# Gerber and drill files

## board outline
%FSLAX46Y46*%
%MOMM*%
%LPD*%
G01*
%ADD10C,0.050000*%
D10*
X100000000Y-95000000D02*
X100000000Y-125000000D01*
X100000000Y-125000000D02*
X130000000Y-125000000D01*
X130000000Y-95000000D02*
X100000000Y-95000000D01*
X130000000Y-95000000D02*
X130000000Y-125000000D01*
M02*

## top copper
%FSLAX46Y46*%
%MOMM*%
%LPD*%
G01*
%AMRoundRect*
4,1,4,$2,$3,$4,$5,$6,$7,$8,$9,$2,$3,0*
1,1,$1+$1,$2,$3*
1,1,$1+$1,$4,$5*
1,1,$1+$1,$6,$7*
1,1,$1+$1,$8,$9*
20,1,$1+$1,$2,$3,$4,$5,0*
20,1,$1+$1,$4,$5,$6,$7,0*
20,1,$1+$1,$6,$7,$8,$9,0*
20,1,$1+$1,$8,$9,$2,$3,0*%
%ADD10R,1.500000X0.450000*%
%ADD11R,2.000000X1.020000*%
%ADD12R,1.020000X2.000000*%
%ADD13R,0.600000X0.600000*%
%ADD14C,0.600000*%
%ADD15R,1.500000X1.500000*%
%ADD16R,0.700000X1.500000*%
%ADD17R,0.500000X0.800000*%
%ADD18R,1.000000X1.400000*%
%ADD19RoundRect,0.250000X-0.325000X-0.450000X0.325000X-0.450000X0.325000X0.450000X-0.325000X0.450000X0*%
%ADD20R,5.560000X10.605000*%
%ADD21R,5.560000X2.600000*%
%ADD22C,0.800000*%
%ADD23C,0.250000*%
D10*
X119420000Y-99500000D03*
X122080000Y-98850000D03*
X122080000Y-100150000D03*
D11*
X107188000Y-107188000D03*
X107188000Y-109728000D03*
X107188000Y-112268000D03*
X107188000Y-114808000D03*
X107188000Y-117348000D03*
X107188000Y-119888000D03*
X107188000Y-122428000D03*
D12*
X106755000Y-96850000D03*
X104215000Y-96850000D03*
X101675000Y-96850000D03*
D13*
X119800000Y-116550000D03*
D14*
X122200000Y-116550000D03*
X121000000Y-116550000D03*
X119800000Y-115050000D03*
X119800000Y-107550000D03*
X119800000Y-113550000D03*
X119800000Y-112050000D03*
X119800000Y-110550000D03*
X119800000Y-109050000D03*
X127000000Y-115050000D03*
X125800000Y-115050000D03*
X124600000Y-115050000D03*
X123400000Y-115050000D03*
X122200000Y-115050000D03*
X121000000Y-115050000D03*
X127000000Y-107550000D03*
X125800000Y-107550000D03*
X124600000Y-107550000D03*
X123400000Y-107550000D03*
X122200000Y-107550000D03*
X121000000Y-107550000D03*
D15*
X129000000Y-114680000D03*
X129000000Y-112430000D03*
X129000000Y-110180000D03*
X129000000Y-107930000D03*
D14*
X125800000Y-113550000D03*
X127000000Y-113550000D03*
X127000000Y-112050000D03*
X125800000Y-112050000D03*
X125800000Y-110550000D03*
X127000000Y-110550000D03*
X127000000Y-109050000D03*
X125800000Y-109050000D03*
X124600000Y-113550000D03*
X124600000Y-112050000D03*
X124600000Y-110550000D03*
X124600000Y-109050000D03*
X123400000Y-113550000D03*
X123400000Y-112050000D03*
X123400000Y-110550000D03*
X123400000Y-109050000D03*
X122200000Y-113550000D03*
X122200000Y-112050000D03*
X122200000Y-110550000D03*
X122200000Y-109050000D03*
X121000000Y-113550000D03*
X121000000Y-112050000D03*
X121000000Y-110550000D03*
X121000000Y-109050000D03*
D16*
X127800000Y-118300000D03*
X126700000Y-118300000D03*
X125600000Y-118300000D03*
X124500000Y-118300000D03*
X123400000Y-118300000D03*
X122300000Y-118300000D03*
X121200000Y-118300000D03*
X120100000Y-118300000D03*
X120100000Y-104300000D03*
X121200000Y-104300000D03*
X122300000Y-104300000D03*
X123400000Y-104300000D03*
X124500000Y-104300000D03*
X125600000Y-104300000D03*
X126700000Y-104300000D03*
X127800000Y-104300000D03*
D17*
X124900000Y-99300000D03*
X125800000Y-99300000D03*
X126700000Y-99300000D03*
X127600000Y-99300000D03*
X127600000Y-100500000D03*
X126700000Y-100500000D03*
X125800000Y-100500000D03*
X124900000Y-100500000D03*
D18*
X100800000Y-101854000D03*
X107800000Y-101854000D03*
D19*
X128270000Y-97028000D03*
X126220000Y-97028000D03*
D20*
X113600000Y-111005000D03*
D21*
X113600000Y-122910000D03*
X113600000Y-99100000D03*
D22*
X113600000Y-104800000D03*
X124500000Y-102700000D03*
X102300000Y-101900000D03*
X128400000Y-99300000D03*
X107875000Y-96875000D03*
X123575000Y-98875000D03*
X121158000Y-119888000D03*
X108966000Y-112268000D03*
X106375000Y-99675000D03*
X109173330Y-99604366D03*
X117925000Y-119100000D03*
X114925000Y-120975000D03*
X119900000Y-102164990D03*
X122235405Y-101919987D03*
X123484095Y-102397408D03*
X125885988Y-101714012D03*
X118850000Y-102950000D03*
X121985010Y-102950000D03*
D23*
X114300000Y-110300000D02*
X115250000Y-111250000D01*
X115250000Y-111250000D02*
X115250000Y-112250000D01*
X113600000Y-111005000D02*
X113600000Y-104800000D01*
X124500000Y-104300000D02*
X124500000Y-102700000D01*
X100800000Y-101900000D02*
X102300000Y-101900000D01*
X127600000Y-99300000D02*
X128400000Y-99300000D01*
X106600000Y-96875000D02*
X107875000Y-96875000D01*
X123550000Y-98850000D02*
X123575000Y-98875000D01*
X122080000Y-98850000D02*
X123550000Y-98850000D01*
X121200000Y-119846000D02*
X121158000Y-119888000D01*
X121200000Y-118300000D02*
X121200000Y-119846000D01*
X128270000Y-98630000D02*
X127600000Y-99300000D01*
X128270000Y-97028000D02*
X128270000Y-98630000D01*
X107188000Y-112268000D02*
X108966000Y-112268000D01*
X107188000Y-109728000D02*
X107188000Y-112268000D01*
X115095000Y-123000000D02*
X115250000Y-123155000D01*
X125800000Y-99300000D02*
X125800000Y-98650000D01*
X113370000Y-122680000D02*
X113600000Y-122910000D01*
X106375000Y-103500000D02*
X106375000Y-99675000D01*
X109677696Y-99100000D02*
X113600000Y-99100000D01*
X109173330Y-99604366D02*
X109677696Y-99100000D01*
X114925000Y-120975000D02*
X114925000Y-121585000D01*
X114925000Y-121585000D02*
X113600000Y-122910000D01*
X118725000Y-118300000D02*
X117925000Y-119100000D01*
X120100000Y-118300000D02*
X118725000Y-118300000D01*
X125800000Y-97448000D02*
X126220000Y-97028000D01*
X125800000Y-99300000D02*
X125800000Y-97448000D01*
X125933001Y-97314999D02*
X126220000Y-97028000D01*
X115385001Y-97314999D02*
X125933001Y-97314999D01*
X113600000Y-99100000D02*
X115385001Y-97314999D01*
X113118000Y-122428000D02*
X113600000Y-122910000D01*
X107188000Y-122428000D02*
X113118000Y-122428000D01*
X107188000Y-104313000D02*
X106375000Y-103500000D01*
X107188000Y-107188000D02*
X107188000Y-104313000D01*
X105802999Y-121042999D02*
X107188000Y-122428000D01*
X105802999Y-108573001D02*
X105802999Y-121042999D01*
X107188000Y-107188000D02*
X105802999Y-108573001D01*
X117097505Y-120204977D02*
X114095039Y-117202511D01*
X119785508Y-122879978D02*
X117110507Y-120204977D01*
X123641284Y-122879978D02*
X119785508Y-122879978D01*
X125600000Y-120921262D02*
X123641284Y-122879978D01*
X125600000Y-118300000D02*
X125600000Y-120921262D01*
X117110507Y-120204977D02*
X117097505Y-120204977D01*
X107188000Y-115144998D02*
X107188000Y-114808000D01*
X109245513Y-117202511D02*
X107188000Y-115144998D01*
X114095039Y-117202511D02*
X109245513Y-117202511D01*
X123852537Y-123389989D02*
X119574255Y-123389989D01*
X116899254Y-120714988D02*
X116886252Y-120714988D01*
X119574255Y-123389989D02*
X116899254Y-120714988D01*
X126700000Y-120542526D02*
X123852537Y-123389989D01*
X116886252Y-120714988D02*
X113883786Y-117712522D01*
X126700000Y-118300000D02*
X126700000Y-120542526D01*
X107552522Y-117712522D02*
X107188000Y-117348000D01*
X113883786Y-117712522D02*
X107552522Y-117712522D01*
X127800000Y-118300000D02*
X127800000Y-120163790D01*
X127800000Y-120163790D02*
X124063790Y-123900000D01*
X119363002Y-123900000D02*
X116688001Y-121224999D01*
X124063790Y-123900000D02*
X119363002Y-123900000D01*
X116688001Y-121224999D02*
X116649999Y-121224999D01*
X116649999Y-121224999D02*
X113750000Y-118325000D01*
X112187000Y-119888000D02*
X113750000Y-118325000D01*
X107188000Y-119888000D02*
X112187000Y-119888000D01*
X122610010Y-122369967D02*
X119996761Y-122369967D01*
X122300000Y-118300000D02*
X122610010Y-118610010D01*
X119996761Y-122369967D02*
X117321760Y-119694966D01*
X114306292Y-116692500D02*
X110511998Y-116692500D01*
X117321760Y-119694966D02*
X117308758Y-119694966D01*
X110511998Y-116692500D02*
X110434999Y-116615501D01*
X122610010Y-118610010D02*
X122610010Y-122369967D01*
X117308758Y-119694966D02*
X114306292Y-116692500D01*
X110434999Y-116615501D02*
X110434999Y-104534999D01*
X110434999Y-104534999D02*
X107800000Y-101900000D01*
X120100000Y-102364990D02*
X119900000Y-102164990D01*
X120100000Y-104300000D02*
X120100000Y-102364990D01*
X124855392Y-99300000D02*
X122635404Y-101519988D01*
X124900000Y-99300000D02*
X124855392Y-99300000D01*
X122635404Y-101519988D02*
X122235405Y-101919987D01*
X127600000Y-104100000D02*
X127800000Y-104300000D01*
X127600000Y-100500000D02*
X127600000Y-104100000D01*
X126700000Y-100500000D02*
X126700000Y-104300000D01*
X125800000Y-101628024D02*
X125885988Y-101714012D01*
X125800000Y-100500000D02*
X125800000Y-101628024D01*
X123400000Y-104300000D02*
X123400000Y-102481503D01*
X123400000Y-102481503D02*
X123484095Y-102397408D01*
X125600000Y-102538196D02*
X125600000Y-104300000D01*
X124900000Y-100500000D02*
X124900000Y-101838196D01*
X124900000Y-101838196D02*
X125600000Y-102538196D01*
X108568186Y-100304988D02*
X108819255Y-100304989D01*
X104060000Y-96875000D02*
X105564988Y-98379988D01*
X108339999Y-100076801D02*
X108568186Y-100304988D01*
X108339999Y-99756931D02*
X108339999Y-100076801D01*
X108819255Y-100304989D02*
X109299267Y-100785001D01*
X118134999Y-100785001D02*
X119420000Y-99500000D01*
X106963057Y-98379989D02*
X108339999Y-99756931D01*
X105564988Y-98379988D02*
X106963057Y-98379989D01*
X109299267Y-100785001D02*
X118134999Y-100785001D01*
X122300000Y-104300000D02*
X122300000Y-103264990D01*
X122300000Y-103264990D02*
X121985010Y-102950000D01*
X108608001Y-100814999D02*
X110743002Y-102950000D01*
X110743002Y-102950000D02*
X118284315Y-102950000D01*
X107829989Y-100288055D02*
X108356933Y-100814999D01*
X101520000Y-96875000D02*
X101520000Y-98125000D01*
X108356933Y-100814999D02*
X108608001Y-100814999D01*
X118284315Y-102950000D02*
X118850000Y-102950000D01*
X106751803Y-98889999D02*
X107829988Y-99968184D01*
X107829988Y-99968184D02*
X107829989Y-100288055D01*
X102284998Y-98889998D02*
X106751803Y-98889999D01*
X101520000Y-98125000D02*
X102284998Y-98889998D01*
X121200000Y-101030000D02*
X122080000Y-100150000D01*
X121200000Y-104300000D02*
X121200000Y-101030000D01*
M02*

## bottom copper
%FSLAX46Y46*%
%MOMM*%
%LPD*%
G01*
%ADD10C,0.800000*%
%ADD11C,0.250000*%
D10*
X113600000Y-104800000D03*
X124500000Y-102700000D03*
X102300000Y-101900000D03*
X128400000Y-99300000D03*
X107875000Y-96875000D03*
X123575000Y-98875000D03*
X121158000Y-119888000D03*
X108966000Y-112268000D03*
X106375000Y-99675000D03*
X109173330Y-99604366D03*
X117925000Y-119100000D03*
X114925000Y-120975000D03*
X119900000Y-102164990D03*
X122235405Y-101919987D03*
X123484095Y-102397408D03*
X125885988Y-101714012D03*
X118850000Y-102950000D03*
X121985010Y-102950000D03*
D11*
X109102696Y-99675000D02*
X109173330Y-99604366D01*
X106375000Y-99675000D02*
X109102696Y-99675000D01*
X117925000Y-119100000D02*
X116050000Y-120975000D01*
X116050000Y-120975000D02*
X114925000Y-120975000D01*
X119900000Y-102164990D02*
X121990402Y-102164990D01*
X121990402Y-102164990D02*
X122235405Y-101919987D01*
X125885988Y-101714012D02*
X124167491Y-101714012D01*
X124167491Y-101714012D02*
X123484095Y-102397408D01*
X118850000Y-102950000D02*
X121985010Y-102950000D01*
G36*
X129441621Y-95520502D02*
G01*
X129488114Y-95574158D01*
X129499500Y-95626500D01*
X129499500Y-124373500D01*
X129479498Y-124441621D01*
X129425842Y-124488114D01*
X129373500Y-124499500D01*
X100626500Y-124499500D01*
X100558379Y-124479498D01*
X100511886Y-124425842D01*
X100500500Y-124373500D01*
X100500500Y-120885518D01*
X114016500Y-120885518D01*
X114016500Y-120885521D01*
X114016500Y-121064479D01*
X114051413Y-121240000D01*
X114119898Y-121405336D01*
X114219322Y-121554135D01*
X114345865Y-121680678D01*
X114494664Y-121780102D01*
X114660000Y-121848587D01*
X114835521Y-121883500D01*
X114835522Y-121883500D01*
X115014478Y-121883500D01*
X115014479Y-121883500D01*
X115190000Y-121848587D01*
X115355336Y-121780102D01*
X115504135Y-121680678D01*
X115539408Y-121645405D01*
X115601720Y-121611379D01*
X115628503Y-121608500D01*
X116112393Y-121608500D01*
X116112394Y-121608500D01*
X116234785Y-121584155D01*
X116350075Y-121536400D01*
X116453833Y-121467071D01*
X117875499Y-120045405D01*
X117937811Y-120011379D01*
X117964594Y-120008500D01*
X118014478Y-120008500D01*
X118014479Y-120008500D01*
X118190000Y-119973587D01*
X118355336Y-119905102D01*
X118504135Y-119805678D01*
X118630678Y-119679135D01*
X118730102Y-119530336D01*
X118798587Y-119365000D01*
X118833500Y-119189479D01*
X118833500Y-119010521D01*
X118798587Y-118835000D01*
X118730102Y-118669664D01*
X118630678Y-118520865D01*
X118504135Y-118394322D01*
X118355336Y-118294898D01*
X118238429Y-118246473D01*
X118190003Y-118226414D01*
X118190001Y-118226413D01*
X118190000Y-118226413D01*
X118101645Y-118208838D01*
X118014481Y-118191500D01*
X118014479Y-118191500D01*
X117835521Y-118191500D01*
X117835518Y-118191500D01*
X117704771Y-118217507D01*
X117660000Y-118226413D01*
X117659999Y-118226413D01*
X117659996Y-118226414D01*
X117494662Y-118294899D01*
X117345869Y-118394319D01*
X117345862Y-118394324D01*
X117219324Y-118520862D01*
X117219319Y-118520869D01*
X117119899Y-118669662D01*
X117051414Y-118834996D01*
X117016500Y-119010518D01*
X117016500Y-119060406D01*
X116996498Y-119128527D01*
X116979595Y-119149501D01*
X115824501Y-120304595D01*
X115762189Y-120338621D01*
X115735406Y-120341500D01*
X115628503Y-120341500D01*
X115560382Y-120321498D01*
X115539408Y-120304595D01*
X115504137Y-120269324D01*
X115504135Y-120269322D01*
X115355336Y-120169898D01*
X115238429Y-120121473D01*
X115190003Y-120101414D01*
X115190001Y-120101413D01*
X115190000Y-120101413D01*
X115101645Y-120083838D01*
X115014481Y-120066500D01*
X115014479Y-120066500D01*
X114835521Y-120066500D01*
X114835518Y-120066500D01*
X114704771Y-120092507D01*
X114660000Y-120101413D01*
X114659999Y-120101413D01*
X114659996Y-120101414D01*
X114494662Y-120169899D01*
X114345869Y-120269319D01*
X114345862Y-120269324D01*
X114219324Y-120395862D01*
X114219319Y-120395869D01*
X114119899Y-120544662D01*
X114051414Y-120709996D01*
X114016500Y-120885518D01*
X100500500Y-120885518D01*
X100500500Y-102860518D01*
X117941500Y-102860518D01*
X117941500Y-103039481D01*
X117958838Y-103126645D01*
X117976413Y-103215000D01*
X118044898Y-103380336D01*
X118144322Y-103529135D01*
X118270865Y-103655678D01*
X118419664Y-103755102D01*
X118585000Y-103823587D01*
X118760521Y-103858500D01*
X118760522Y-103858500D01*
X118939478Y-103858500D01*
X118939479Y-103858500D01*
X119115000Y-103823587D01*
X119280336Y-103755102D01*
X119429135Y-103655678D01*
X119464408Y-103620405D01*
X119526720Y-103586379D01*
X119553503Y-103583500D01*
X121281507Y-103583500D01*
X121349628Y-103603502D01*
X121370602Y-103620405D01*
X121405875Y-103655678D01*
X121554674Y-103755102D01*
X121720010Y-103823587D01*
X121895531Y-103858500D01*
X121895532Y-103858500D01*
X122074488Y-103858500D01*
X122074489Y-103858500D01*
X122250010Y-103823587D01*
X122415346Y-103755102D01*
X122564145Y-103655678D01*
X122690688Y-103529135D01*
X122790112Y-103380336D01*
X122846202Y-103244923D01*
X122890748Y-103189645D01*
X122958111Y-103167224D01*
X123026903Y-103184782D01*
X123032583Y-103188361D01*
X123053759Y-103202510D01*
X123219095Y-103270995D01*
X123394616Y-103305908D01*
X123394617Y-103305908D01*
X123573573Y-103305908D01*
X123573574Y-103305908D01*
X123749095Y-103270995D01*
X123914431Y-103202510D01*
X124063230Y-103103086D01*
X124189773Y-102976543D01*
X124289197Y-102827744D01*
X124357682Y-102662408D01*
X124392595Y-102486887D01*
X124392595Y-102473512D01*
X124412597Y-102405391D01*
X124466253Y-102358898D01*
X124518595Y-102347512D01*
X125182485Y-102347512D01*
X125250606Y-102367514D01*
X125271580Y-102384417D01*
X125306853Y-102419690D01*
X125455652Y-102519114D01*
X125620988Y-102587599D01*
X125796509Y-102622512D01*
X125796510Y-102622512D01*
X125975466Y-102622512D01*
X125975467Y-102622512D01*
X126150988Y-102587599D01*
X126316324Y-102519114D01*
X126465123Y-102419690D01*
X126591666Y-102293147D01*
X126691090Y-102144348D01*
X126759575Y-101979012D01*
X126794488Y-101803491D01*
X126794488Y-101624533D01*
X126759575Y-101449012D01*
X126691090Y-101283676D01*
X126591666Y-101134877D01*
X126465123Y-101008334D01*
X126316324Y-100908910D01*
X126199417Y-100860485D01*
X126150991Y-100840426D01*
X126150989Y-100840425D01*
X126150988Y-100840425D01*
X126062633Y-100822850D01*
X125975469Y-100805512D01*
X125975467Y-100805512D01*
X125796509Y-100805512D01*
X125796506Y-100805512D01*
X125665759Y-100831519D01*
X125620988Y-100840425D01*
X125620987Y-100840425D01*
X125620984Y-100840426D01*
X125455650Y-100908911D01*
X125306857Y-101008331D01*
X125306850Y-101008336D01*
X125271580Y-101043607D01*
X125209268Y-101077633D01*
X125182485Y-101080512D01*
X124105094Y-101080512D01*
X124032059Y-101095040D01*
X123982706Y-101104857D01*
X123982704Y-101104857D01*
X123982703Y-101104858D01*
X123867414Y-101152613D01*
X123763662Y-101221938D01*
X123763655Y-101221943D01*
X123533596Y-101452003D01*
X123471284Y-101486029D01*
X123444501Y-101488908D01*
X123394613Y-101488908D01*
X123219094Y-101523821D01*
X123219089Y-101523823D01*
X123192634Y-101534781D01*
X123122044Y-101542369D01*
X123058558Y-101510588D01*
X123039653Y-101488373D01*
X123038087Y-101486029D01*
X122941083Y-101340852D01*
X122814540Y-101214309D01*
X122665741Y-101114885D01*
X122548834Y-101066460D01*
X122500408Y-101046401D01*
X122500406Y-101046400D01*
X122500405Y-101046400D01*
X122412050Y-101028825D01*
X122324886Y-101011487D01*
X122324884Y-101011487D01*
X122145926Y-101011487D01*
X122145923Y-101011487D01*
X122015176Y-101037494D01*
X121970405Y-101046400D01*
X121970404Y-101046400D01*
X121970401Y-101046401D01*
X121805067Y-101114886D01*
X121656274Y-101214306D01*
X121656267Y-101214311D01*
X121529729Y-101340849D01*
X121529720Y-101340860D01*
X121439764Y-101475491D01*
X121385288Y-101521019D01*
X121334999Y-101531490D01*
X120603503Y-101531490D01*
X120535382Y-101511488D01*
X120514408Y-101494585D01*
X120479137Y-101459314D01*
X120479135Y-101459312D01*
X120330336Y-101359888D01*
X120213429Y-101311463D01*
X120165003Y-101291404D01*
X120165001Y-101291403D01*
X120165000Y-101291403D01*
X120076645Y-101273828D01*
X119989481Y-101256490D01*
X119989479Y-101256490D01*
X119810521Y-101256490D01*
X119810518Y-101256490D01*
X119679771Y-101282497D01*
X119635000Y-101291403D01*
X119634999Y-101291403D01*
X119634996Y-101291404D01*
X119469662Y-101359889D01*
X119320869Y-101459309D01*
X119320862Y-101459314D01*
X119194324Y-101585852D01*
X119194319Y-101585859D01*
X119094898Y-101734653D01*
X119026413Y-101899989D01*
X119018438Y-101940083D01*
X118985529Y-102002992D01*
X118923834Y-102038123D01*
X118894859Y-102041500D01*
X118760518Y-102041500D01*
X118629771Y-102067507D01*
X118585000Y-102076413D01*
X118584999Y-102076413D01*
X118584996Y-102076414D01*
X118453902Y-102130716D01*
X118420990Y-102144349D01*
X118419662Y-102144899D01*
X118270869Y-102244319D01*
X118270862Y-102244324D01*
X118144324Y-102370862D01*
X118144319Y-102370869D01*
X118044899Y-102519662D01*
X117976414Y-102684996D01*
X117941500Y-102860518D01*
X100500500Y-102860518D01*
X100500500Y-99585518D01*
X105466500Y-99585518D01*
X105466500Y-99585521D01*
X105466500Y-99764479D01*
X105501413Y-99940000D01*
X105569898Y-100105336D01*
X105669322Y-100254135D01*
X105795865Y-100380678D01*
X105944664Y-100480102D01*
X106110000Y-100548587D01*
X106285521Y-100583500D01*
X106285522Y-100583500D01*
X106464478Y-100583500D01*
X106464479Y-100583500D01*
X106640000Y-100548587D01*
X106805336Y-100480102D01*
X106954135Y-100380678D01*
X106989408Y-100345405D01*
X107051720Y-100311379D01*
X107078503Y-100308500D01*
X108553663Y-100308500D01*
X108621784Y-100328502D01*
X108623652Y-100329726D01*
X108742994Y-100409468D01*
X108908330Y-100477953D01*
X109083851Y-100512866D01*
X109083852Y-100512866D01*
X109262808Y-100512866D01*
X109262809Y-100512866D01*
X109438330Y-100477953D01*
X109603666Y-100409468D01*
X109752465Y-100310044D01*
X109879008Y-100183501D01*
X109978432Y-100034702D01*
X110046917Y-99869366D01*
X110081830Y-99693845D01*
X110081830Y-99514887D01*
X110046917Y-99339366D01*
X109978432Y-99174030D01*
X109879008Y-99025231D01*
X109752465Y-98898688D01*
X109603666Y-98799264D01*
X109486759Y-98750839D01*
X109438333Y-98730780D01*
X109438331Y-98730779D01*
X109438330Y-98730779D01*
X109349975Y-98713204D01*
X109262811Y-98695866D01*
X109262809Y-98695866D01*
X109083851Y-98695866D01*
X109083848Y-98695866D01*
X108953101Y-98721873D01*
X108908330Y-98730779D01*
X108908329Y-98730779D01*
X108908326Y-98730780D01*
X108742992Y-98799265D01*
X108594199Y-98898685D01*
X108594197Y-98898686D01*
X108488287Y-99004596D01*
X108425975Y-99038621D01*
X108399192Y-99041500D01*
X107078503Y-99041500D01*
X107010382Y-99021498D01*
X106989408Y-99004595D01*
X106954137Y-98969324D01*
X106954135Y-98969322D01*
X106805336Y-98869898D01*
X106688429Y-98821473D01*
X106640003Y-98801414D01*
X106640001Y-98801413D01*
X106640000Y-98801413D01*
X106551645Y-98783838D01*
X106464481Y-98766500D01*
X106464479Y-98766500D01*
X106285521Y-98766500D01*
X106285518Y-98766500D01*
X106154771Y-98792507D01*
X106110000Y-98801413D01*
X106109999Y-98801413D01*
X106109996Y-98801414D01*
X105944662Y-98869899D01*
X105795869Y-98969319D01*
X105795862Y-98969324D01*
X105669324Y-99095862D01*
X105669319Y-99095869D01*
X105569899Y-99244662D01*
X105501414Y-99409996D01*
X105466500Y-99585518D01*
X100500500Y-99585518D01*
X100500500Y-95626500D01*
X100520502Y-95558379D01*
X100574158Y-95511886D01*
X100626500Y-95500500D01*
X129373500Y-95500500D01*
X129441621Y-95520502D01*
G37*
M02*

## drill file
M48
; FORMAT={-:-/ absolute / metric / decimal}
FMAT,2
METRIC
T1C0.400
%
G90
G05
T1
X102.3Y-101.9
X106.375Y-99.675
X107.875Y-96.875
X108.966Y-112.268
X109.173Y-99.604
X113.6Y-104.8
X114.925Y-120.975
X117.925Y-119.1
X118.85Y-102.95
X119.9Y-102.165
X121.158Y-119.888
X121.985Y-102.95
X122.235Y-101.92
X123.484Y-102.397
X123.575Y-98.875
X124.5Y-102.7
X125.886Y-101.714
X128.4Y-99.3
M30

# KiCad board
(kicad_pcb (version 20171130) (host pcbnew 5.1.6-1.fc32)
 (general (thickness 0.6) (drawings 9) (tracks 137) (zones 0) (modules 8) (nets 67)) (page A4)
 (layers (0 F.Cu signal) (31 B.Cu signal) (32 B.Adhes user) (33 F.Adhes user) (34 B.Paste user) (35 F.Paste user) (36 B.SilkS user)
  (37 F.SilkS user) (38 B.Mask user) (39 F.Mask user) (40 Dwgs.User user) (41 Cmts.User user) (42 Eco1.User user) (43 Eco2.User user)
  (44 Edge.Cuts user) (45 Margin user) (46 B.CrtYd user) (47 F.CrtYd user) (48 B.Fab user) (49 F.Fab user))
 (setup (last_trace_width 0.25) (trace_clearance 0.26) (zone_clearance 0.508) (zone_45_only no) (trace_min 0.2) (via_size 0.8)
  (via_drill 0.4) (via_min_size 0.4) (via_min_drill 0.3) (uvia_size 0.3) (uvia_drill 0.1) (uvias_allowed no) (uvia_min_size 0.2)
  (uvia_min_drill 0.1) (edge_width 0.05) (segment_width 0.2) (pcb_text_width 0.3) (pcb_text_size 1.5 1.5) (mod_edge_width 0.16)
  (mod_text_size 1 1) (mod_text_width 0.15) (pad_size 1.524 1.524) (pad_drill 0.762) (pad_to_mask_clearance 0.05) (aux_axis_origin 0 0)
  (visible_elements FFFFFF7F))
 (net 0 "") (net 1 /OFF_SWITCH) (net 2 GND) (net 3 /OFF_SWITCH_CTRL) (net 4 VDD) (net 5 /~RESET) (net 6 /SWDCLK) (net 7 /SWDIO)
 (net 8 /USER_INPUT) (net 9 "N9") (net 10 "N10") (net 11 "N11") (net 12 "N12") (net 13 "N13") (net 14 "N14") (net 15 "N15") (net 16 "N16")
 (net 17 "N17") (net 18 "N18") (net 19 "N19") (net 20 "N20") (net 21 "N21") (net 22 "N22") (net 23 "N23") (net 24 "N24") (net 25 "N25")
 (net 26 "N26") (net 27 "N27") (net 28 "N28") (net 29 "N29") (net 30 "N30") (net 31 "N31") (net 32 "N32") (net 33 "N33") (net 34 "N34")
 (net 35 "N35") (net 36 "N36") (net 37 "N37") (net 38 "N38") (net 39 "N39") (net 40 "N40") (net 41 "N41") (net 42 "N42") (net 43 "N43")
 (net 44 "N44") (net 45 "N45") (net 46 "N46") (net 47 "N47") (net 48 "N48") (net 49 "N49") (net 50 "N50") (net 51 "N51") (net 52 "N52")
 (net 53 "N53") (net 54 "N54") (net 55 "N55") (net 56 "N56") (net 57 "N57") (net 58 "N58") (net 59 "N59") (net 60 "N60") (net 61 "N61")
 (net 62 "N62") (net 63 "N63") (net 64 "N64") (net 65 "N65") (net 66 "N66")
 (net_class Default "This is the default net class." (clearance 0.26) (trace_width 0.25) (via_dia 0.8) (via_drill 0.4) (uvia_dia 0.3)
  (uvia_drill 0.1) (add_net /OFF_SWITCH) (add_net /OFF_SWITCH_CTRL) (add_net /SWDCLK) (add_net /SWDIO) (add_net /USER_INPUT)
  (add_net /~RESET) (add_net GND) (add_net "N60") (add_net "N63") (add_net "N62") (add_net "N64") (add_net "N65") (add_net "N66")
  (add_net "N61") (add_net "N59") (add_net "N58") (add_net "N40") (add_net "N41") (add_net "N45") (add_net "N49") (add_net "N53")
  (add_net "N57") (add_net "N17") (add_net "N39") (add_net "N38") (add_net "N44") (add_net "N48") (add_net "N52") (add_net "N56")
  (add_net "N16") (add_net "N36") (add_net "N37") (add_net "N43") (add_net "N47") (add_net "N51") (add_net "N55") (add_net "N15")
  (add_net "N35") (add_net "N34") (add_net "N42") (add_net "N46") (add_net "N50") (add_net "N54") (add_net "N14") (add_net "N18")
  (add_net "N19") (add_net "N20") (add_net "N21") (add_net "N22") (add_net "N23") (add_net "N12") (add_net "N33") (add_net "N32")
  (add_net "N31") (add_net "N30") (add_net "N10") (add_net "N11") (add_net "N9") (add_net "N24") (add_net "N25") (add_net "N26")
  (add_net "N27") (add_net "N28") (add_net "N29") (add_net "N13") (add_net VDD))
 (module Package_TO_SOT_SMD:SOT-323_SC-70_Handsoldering (layer F.Cu) (at 120.75 99.5 180)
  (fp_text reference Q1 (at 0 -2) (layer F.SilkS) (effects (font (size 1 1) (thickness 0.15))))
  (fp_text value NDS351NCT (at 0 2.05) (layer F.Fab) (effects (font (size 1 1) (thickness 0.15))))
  (pad 3 smd rect (at 1.33 0 90) (size 0.45 1.5) (layers F.Cu F.Paste F.Mask) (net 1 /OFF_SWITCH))
  (pad 2 smd rect (at -1.33 0.65 90) (size 0.45 1.5) (layers F.Cu F.Paste F.Mask) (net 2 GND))
  (pad 1 smd rect (at -1.33 -0.65 90) (size 0.45 1.5) (layers F.Cu F.Paste F.Mask) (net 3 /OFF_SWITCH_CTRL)))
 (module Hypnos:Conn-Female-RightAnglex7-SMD (layer F.Cu) (at 107.188 122.428 90)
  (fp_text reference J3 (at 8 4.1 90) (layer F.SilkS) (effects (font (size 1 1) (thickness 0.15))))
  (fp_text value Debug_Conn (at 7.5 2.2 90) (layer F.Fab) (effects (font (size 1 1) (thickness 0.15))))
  (pad 7 smd rect (at 15.24 0 90) (size 1.02 2) (layers F.Cu F.Paste F.Mask) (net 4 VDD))
  (pad 6 smd rect (at 12.7 0 90) (size 1.02 2) (layers F.Cu F.Paste F.Mask) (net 2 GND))
  (pad 5 smd rect (at 10.16 0 90) (size 1.02 2) (layers F.Cu F.Paste F.Mask) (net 2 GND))
  (pad 4 smd rect (at 7.62 0 90) (size 1.02 2) (layers F.Cu F.Paste F.Mask) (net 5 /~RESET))
  (pad 3 smd rect (at 5.08 0 90) (size 1.02 2) (layers F.Cu F.Paste F.Mask) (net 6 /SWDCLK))
  (pad 2 smd rect (at 2.54 0 90) (size 1.02 2) (layers F.Cu F.Paste F.Mask) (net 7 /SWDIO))
  (pad 1 smd rect (at 0 0 90) (size 1.02 2) (layers F.Cu F.Paste F.Mask) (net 4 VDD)))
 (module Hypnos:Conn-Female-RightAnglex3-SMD (layer F.Cu) (at 101.675 96.85)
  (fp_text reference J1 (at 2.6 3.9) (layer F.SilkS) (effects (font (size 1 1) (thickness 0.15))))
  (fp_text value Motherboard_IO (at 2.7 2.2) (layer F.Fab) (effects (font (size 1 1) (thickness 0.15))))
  (pad 3 smd rect (at 5.08 0) (size 1.02 2) (layers F.Cu F.Paste F.Mask) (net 2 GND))
  (pad 2 smd rect (at 2.54 0) (size 1.02 2) (layers F.Cu F.Paste F.Mask) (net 1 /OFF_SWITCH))
  (pad 1 smd rect (at 0 0) (size 1.02 2) (layers F.Cu F.Paste F.Mask) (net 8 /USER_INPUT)))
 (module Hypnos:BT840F (layer F.Cu) (at 129.4 110.8 270)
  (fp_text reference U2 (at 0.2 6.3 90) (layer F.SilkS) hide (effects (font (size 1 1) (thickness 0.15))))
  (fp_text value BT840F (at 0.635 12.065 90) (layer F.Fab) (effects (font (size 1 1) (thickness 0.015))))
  (pad F6 smd rect (at 5.75 9.6 270) (size 0.6 0.6) (layers F.Cu F.Paste F.Mask) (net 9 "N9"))
  (pad F4 smd circle (at 5.75 7.2 270) (size 0.6 0.6) (layers F.Cu F.Paste F.Mask) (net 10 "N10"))
  (pad F5 smd circle (at 5.75 8.4 270) (size 0.6 0.6) (layers F.Cu F.Paste F.Mask) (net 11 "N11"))
  (pad E6 smd circle (at 4.25 9.6 270) (size 0.6 0.6) (layers F.Cu F.Paste F.Mask) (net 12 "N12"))
  (pad Z6 smd circle (at -3.25 9.6 270) (size 0.6 0.6) (layers F.Cu F.Paste F.Mask) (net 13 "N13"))
  (pad D6 smd circle (at 2.75 9.6 270) (size 0.6 0.6) (layers F.Cu F.Paste F.Mask) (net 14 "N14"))
  (pad C6 smd circle (at 1.25 9.6 270) (size 0.6 0.6) (layers F.Cu F.Paste F.Mask) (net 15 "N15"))
  (pad B6 smd circle (at -0.25 9.6 270) (size 0.6 0.6) (layers F.Cu F.Paste F.Mask) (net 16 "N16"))
  (pad A6 smd circle (at -1.75 9.6 270) (size 0.6 0.6) (layers F.Cu F.Paste F.Mask) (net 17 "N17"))
  (pad E0 smd circle (at 4.25 2.4 270) (size 0.6 0.6) (layers F.Cu F.Paste F.Mask) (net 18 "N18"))
  (pad E1 smd circle (at 4.25 3.6 270) (size 0.6 0.6) (layers F.Cu F.Paste F.Mask) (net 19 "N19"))
  (pad E2 smd circle (at 4.25 4.8 270) (size 0.6 0.6) (layers F.Cu F.Paste F.Mask) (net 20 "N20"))
  (pad E3 smd circle (at 4.25 6 270) (size 0.6 0.6) (layers F.Cu F.Paste F.Mask) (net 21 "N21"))
  (pad E4 smd circle (at 4.25 7.2 270) (size 0.6 0.6) (layers F.Cu F.Paste F.Mask) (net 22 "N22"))
  (pad E5 smd circle (at 4.25 8.4 270) (size 0.6 0.6) (layers F.Cu F.Paste F.Mask) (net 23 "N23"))
  (pad Z0 smd circle (at -3.25 2.4 270) (size 0.6 0.6) (layers F.Cu F.Paste F.Mask) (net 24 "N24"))
  (pad Z1 smd circle (at -3.25 3.6 270) (size 0.6 0.6) (layers F.Cu F.Paste F.Mask) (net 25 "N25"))
  (pad Z2 smd circle (at -3.25 4.8 270) (size 0.6 0.6) (layers F.Cu F.Paste F.Mask) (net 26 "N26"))
  (pad Z3 smd circle (at -3.25 6 270) (size 0.6 0.6) (layers F.Cu F.Paste F.Mask) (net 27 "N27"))
  (pad Z4 smd circle (at -3.25 7.2 270) (size 0.6 0.6) (layers F.Cu F.Paste F.Mask) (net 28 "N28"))
  (pad Z5 smd circle (at -3.25 8.4 270) (size 0.6 0.6) (layers F.Cu F.Paste F.Mask) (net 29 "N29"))
  (pad F3 smd rect (at 3.88 0.4 270) (size 1.5 1.5) (layers F.Cu F.Paste F.Mask) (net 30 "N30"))
  (pad F2 smd rect (at 1.63 0.4 270) (size 1.5 1.5) (layers F.Cu F.Paste F.Mask) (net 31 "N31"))
  (pad F1 smd rect (at -0.62 0.4 270) (size 1.5 1.5) (layers F.Cu F.Paste F.Mask) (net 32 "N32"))
  (pad F0 smd rect (at -2.87 0.4 270) (size 1.5 1.5) (layers F.Cu F.Paste F.Mask) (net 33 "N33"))
  (pad D1 smd circle (at 2.75 3.6 270) (size 0.6 0.6) (layers F.Cu F.Paste F.Mask) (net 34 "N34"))
  (pad D0 smd circle (at 2.75 2.4 270) (size 0.6 0.6) (layers F.Cu F.Paste F.Mask) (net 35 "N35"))
  (pad C0 smd circle (at 1.25 2.4 270) (size 0.6 0.6) (layers F.Cu F.Paste F.Mask) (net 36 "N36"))
  (pad C1 smd circle (at 1.25 3.6 270) (size 0.6 0.6) (layers F.Cu F.Paste F.Mask) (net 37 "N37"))
  (pad B1 smd circle (at -0.25 3.6 270) (size 0.6 0.6) (layers F.Cu F.Paste F.Mask) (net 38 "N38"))
  (pad B0 smd circle (at -0.25 2.4 270) (size 0.6 0.6) (layers F.Cu F.Paste F.Mask) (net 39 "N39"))
  (pad A0 smd circle (at -1.75 2.4 270) (size 0.6 0.6) (layers F.Cu F.Paste F.Mask) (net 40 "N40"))
  (pad A1 smd circle (at -1.75 3.6 270) (size 0.6 0.6) (layers F.Cu F.Paste F.Mask) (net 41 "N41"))
  (pad D2 smd circle (at 2.75 4.8 270) (size 0.6 0.6) (layers F.Cu F.Paste F.Mask) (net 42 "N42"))
  (pad C2 smd circle (at 1.25 4.8 270) (size 0.6 0.6) (layers F.Cu F.Paste F.Mask) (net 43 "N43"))
  (pad B2 smd circle (at -0.25 4.8 270) (size 0.6 0.6) (layers F.Cu F.Paste F.Mask) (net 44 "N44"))
  (pad A2 smd circle (at -1.75 4.8 270) (size 0.6 0.6) (layers F.Cu F.Paste F.Mask) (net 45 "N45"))
  (pad D3 smd circle (at 2.75 6 270) (size 0.6 0.6) (layers F.Cu F.Paste F.Mask) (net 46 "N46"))
  (pad C3 smd circle (at 1.25 6 270) (size 0.6 0.6) (layers F.Cu F.Paste F.Mask) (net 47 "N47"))
  (pad B3 smd circle (at -0.25 6 270) (size 0.6 0.6) (layers F.Cu F.Paste F.Mask) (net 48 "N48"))
  (pad A3 smd circle (at -1.75 6 270) (size 0.6 0.6) (layers F.Cu F.Paste F.Mask) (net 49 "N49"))
  (pad D4 smd circle (at 2.75 7.2 270) (size 0.6 0.6) (layers F.Cu F.Paste F.Mask) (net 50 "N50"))
  (pad C4 smd circle (at 1.25 7.2 270) (size 0.6 0.6) (layers F.Cu F.Paste F.Mask) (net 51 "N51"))
  (pad B4 smd circle (at -0.25 7.2 270) (size 0.6 0.6) (layers F.Cu F.Paste F.Mask) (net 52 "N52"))
  (pad A4 smd circle (at -1.75 7.2 270) (size 0.6 0.6) (layers F.Cu F.Paste F.Mask) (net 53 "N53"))
  (pad D5 smd circle (at 2.75 8.4 270) (size 0.6 0.6) (layers F.Cu F.Paste F.Mask) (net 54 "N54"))
  (pad C5 smd circle (at 1.25 8.4 270) (size 0.6 0.6) (layers F.Cu F.Paste F.Mask) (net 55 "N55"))
  (pad B5 smd circle (at -0.25 8.4 270) (size 0.6 0.6) (layers F.Cu F.Paste F.Mask) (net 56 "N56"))
  (pad A5 smd circle (at -1.75 8.4 270) (size 0.6 0.6) (layers F.Cu F.Paste F.Mask) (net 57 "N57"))
  (pad 16 smd rect (at 7.5 1.6 270) (size 1.5 0.7) (layers F.Cu F.Paste F.Mask) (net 7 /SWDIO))
  (pad 15 smd rect (at 7.5 2.7 270) (size 1.5 0.7) (layers F.Cu F.Paste F.Mask) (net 6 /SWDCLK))
  (pad 14 smd rect (at 7.5 3.8 270) (size 1.5 0.7) (layers F.Cu F.Paste F.Mask) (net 5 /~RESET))
  (pad 13 smd rect (at 7.5 4.9 270) (size 1.5 0.7) (layers F.Cu F.Paste F.Mask) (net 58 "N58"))
  (pad 12 smd rect (at 7.5 6 270) (size 1.5 0.7) (layers F.Cu F.Paste F.Mask) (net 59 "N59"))
  (pad 11 smd rect (at 7.5 7.1 270) (size 1.5 0.7) (layers F.Cu F.Paste F.Mask) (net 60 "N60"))
  (pad 10 smd rect (at 7.5 8.2 270) (size 1.5 0.7) (layers F.Cu F.Paste F.Mask) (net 2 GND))
  (pad 9 smd rect (at 7.5 9.3 270) (size 1.5 0.7) (layers F.Cu F.Paste F.Mask) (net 4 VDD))
  (pad 8 smd rect (at -6.5 9.3 270) (size 1.5 0.7) (layers F.Cu F.Paste F.Mask) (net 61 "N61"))
  (pad 7 smd rect (at -6.5 8.2 270) (size 1.5 0.7) (layers F.Cu F.Paste F.Mask) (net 3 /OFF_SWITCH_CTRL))
  (pad 6 smd rect (at -6.5 7.1 270) (size 1.5 0.7) (layers F.Cu F.Paste F.Mask) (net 8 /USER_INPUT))
  (pad 5 smd rect (at -6.5 6 270) (size 1.5 0.7) (layers F.Cu F.Paste F.Mask) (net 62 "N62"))
  (pad 4 smd rect (at -6.5 4.9 270) (size 1.5 0.7) (layers F.Cu F.Paste F.Mask) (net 2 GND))
  (pad 3 smd rect (at -6.5 3.8 270) (size 1.5 0.7) (layers F.Cu F.Paste F.Mask) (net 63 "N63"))
  (pad 2 smd rect (at -6.5 2.7 270) (size 1.5 0.7) (layers F.Cu F.Paste F.Mask) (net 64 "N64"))
  (pad 1 smd rect (at -6.5 1.6 270) (size 1.5 0.7) (layers F.Cu F.Paste F.Mask) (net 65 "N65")))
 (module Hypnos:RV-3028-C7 (layer F.Cu) (at 126.25 99.9 90)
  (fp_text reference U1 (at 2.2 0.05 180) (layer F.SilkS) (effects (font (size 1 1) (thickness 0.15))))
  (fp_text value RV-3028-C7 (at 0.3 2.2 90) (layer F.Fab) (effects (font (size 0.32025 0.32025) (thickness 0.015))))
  (pad 8 smd rect (at 0.6 -1.35 90) (size 0.8 0.5) (layers F.Cu F.Paste F.Mask) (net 61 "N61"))
  (pad 7 smd rect (at 0.6 -0.45 90) (size 0.8 0.5) (layers F.Cu F.Paste F.Mask) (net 4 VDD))
  (pad 6 smd rect (at 0.6 0.45 90) (size 0.8 0.5) (layers F.Cu F.Paste F.Mask) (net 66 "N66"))
  (pad 5 smd rect (at 0.6 1.35 90) (size 0.8 0.5) (layers F.Cu F.Paste F.Mask) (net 2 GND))
  (pad 4 smd rect (at -0.6 1.35 90) (size 0.8 0.5) (layers F.Cu F.Paste F.Mask) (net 65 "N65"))
  (pad 3 smd rect (at -0.6 0.45 90) (size 0.8 0.5) (layers F.Cu F.Paste F.Mask) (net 64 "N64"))
  (pad 2 smd rect (at -0.6 -0.45 90) (size 0.8 0.5) (layers F.Cu F.Paste F.Mask) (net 62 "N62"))
  (pad 1 smd rect (at -0.6 -1.35 90) (size 0.8 0.5) (layers F.Cu F.Paste F.Mask) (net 63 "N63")))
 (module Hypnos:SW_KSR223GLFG (layer F.Cu) (at 104.3 101.854 180)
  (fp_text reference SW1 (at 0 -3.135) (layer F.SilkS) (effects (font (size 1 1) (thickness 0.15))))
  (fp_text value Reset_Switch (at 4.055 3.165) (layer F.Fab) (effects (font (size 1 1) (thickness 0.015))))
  (pad 2 smd rect (at 3.5 0 180) (size 1 1.4) (layers F.Cu F.Paste F.Mask) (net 2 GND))
  (pad 1 smd rect (at -3.5 0 180) (size 1 1.4) (layers F.Cu F.Paste F.Mask) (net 60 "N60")))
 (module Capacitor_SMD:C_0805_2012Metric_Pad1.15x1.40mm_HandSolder (layer F.Cu) (at 127.245 97.028)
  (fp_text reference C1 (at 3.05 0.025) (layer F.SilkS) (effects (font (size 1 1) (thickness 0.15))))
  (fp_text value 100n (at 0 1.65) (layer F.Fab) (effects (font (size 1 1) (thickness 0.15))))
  (pad 2 smd roundrect (at 1.025 0) (size 1.15 1.4) (layers F.Cu F.Paste F.Mask) (roundrect_rratio 0.217391) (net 2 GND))
  (pad 1 smd roundrect (at -1.025 0) (size 1.15 1.4) (layers F.Cu F.Paste F.Mask) (roundrect_rratio 0.217391) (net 4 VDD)))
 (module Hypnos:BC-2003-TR (layer F.Cu) (at 113.6 111.005 270)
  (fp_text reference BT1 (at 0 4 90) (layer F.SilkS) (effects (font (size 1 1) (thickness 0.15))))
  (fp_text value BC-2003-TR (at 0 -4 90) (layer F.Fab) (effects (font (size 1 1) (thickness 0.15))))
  (pad 2 smd rect (at 0 0 270) (size 10.605 5.56) (layers F.Cu F.Paste F.Mask) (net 2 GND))
  (pad 3 smd rect (at 11.905 0 270) (size 2.6 5.56) (layers F.Cu F.Paste F.Mask) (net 4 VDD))
  (pad 1 smd rect (at -11.905 0 270) (size 2.6 5.56) (layers F.Cu F.Paste F.Mask) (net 4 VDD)))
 (gr_line (start 100 95) (end 100 125) (layer Edge.Cuts) (width 0.05))
 (gr_line (start 100 125) (end 130 125) (layer Edge.Cuts) (width 0.05))
 (gr_line (start 130 95) (end 100 95) (layer Edge.Cuts) (width 0.05))
 (gr_line (start 130 95) (end 130 125) (layer Edge.Cuts) (width 0.05))
 (segment (start 114.3 110.3) (end 115.25 111.25) (width 0.25) (layer F.Cu) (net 2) (status 30))
 (segment (start 115.25 111.25) (end 115.25 112.25) (width 0.25) (layer F.Cu) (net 2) (status 30))
 (via (at 113.6 104.8) (size 0.8) (drill 0.4) (layers F.Cu B.Cu) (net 2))
 (segment (start 113.6 111.005) (end 113.6 104.8) (width 0.25) (layer F.Cu) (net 2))
 (via (at 124.5 102.7) (size 0.8) (drill 0.4) (layers F.Cu B.Cu) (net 2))
 (segment (start 124.5 104.3) (end 124.5 102.7) (width 0.25) (layer F.Cu) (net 2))
 (via (at 102.3 101.9) (size 0.8) (drill 0.4) (layers F.Cu B.Cu) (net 2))
 (segment (start 100.8 101.9) (end 102.3 101.9) (width 0.25) (layer F.Cu) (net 2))
 (via (at 128.4 99.3) (size 0.8) (drill 0.4) (layers F.Cu B.Cu) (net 2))
 (segment (start 127.6 99.3) (end 128.4 99.3) (width 0.25) (layer F.Cu) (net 2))
 (via (at 107.875 96.875) (size 0.8) (drill 0.4) (layers F.Cu B.Cu) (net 2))
 (segment (start 106.6 96.875) (end 107.875 96.875) (width 0.25) (layer F.Cu) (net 2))
 (via (at 123.575 98.875) (size 0.8) (drill 0.4) (layers F.Cu B.Cu) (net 2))
 (segment (start 123.55 98.85) (end 123.575 98.875) (width 0.25) (layer F.Cu) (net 2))
 (segment (start 122.08 98.85) (end 123.55 98.85) (width 0.25) (layer F.Cu) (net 2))
 (via (at 121.158 119.888) (size 0.8) (drill 0.4) (layers F.Cu B.Cu) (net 2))
 (segment (start 121.2 119.846) (end 121.158 119.888) (width 0.25) (layer F.Cu) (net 2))
 (segment (start 121.2 118.3) (end 121.2 119.846) (width 0.25) (layer F.Cu) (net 2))
 (segment (start 128.27 98.63) (end 127.6 99.3) (width 0.25) (layer F.Cu) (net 2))
 (segment (start 128.27 97.028) (end 128.27 98.63) (width 0.25) (layer F.Cu) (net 2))
 (via (at 108.966 112.268) (size 0.8) (drill 0.4) (layers F.Cu B.Cu) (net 2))
 (segment (start 107.188 112.268) (end 108.966 112.268) (width 0.25) (layer F.Cu) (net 2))
 (segment (start 107.188 109.728) (end 107.188 112.268) (width 0.25) (layer F.Cu) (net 2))
 (segment (start 115.095 123) (end 115.25 123.155) (width 0.25) (layer F.Cu) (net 4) (status 30))
 (segment (start 125.8 99.3) (end 125.8 98.65) (width 0.25) (layer F.Cu) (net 4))
 (segment (start 113.37 122.68) (end 113.6 122.91) (width 0.25) (layer F.Cu) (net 4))
 (via (at 106.375 99.675) (size 0.8) (drill 0.4) (layers F.Cu B.Cu) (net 4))
 (segment (start 106.375 103.5) (end 106.375 99.675) (width 0.25) (layer F.Cu) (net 4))
 (segment (start 109.102696 99.675) (end 109.17333 99.604366) (width 0.25) (layer B.Cu) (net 4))
 (via (at 109.17333 99.604366) (size 0.8) (drill 0.4) (layers F.Cu B.Cu) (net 4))
 (segment (start 106.375 99.675) (end 109.102696 99.675) (width 0.25) (layer B.Cu) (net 4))
 (segment (start 109.677696 99.1) (end 113.6 99.1) (width 0.25) (layer F.Cu) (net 4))
 (segment (start 109.17333 99.604366) (end 109.677696 99.1) (width 0.25) (layer F.Cu) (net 4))
 (via (at 117.925 119.1) (size 0.8) (drill 0.4) (layers F.Cu B.Cu) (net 4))
 (segment (start 114.925 120.975) (end 114.925 121.585) (width 0.25) (layer F.Cu) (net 4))
 (segment (start 114.925 121.585) (end 113.6 122.91) (width 0.25) (layer F.Cu) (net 4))
 (segment (start 117.925 119.1) (end 116.05 120.975) (width 0.25) (layer B.Cu) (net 4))
 (via (at 114.925 120.975) (size 0.8) (drill 0.4) (layers F.Cu B.Cu) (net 4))
 (segment (start 116.05 120.975) (end 114.925 120.975) (width 0.25) (layer B.Cu) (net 4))
 (segment (start 118.725 118.3) (end 117.925 119.1) (width 0.25) (layer F.Cu) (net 4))
 (segment (start 120.1 118.3) (end 118.725 118.3) (width 0.25) (layer F.Cu) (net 4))
 (segment (start 125.8 97.448) (end 126.22 97.028) (width 0.25) (layer F.Cu) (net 4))
 (segment (start 125.8 99.3) (end 125.8 97.448) (width 0.25) (layer F.Cu) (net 4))
 (segment (start 125.933001 97.314999) (end 126.22 97.028) (width 0.25) (layer F.Cu) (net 4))
 (segment (start 115.385001 97.314999) (end 125.933001 97.314999) (width 0.25) (layer F.Cu) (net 4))
 (segment (start 113.6 99.1) (end 115.385001 97.314999) (width 0.25) (layer F.Cu) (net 4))
 (segment (start 113.118 122.428) (end 113.6 122.91) (width 0.25) (layer F.Cu) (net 4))
 (segment (start 107.188 122.428) (end 113.118 122.428) (width 0.25) (layer F.Cu) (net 4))
 (segment (start 107.188 104.313) (end 106.375 103.5) (width 0.25) (layer F.Cu) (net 4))
 (segment (start 107.188 107.188) (end 107.188 104.313) (width 0.25) (layer F.Cu) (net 4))
 (segment (start 105.802999 121.042999) (end 107.188 122.428) (width 0.25) (layer F.Cu) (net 4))
 (segment (start 105.802999 108.573001) (end 105.802999 121.042999) (width 0.25) (layer F.Cu) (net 4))
 (segment (start 107.188 107.188) (end 105.802999 108.573001) (width 0.25) (layer F.Cu) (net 4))
 (segment (start 117.097505 120.204977) (end 114.095039 117.202511) (width 0.25) (layer F.Cu) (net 5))
 (segment (start 119.785508 122.879978) (end 117.110507 120.204977) (width 0.25) (layer F.Cu) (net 5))
 (segment (start 123.641284 122.879978) (end 119.785508 122.879978) (width 0.25) (layer F.Cu) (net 5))
 (segment (start 125.6 120.921262) (end 123.641284 122.879978) (width 0.25) (layer F.Cu) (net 5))
 (segment (start 125.6 118.3) (end 125.6 120.921262) (width 0.25) (layer F.Cu) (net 5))
 (segment (start 117.110507 120.204977) (end 117.097505 120.204977) (width 0.25) (layer F.Cu) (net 5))
 (segment (start 107.188 115.144998) (end 107.188 114.808) (width 0.25) (layer F.Cu) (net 5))
 (segment (start 109.245513 117.202511) (end 107.188 115.144998) (width 0.25) (layer F.Cu) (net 5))
 (segment (start 114.095039 117.202511) (end 109.245513 117.202511) (width 0.25) (layer F.Cu) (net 5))
 (segment (start 123.852537 123.389989) (end 119.574255 123.389989) (width 0.25) (layer F.Cu) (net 6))
 (segment (start 116.899254 120.714988) (end 116.886252 120.714988) (width 0.25) (layer F.Cu) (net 6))
 (segment (start 119.574255 123.389989) (end 116.899254 120.714988) (width 0.25) (layer F.Cu) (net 6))
 (segment (start 126.7 120.542526) (end 123.852537 123.389989) (width 0.25) (layer F.Cu) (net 6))
 (segment (start 116.886252 120.714988) (end 113.883786 117.712522) (width 0.25) (layer F.Cu) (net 6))
 (segment (start 126.7 118.3) (end 126.7 120.542526) (width 0.25) (layer F.Cu) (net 6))
 (segment (start 107.552522 117.712522) (end 107.188 117.348) (width 0.25) (layer F.Cu) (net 6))
 (segment (start 113.883786 117.712522) (end 107.552522 117.712522) (width 0.25) (layer F.Cu) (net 6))
 (segment (start 127.8 118.3) (end 127.8 120.16379) (width 0.25) (layer F.Cu) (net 7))
 (segment (start 127.8 120.16379) (end 124.06379 123.9) (width 0.25) (layer F.Cu) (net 7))
 (segment (start 119.363002 123.9) (end 116.688001 121.224999) (width 0.25) (layer F.Cu) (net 7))
 (segment (start 124.06379 123.9) (end 119.363002 123.9) (width 0.25) (layer F.Cu) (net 7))
 (segment (start 116.688001 121.224999) (end 116.649999 121.224999) (width 0.25) (layer F.Cu) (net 7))
 (segment (start 116.649999 121.224999) (end 113.75 118.325) (width 0.25) (layer F.Cu) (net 7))
 (segment (start 112.187 119.888) (end 113.75 118.325) (width 0.25) (layer F.Cu) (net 7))
 (segment (start 107.188 119.888) (end 112.187 119.888) (width 0.25) (layer F.Cu) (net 7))
 (segment (start 122.61001 122.369967) (end 119.996761 122.369967) (width 0.25) (layer F.Cu) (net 60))
 (segment (start 122.3 118.3) (end 122.61001 118.61001) (width 0.25) (layer F.Cu) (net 60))
 (segment (start 119.996761 122.369967) (end 117.32176 119.694966) (width 0.25) (layer F.Cu) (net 60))
 (segment (start 114.306292 116.6925) (end 110.511998 116.6925) (width 0.25) (layer F.Cu) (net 60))
 (segment (start 117.32176 119.694966) (end 117.308758 119.694966) (width 0.25) (layer F.Cu) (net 60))
 (segment (start 110.511998 116.6925) (end 110.434999 116.615501) (width 0.25) (layer F.Cu) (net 60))
 (segment (start 122.61001 118.61001) (end 122.61001 122.369967) (width 0.25) (layer F.Cu) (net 60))
 (segment (start 117.308758 119.694966) (end 114.306292 116.6925) (width 0.25) (layer F.Cu) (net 60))
 (segment (start 110.434999 116.615501) (end 110.434999 104.534999) (width 0.25) (layer F.Cu) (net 60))
 (segment (start 110.434999 104.534999) (end 107.8 101.9) (width 0.25) (layer F.Cu) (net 60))
 (via (at 119.9 102.16499) (size 0.8) (drill 0.4) (layers F.Cu B.Cu) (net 61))
 (segment (start 120.1 102.36499) (end 119.9 102.16499) (width 0.25) (layer F.Cu) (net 61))
 (segment (start 120.1 104.3) (end 120.1 102.36499) (width 0.25) (layer F.Cu) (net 61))
 (segment (start 124.855392 99.3) (end 122.635404 101.519988) (width 0.25) (layer F.Cu) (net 61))
 (segment (start 124.9 99.3) (end 124.855392 99.3) (width 0.25) (layer F.Cu) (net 61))
 (via (at 122.235405 101.919987) (size 0.8) (drill 0.4) (layers F.Cu B.Cu) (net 61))
 (segment (start 122.635404 101.519988) (end 122.235405 101.919987) (width 0.25) (layer F.Cu) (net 61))
 (segment (start 119.9 102.16499) (end 121.990402 102.16499) (width 0.25) (layer B.Cu) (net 61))
 (segment (start 121.990402 102.16499) (end 122.235405 101.919987) (width 0.25) (layer B.Cu) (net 61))
 (segment (start 127.6 104.1) (end 127.8 104.3) (width 0.25) (layer F.Cu) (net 65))
 (segment (start 127.6 100.5) (end 127.6 104.1) (width 0.25) (layer F.Cu) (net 65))
 (segment (start 126.7 100.5) (end 126.7 104.3) (width 0.25) (layer F.Cu) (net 64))
 (segment (start 125.8 101.628024) (end 125.885988 101.714012) (width 0.25) (layer F.Cu) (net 62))
 (via (at 123.484095 102.397408) (size 0.8) (drill 0.4) (layers F.Cu B.Cu) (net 62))
 (segment (start 125.8 100.5) (end 125.8 101.628024) (width 0.25) (layer F.Cu) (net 62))
 (segment (start 123.4 104.3) (end 123.4 102.481503) (width 0.25) (layer F.Cu) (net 62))
 (via (at 125.885988 101.714012) (size 0.8) (drill 0.4) (layers F.Cu B.Cu) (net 62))
 (segment (start 125.885988 101.714012) (end 124.167491 101.714012) (width 0.25) (layer B.Cu) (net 62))
 (segment (start 124.167491 101.714012) (end 123.484095 102.397408) (width 0.25) (layer B.Cu) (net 62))
 (segment (start 123.4 102.481503) (end 123.484095 102.397408) (width 0.25) (layer F.Cu) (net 62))
 (segment (start 125.6 102.538196) (end 125.6 104.3) (width 0.25) (layer F.Cu) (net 63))
 (segment (start 124.9 100.5) (end 124.9 101.838196) (width 0.25) (layer F.Cu) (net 63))
 (segment (start 124.9 101.838196) (end 125.6 102.538196) (width 0.25) (layer F.Cu) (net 63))
 (segment (start 108.568186 100.304988) (end 108.819255 100.304989) (width 0.25) (layer F.Cu) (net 1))
 (segment (start 104.06 96.875) (end 105.564988 98.379988) (width 0.25) (layer F.Cu) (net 1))
 (segment (start 108.339999 100.076801) (end 108.568186 100.304988) (width 0.25) (layer F.Cu) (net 1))
 (segment (start 108.339999 99.756931) (end 108.339999 100.076801) (width 0.25) (layer F.Cu) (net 1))
 (segment (start 108.819255 100.304989) (end 109.299267 100.785001) (width 0.25) (layer F.Cu) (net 1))
 (segment (start 118.134999 100.785001) (end 119.42 99.5) (width 0.25) (layer F.Cu) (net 1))
 (segment (start 106.963057 98.379989) (end 108.339999 99.756931) (width 0.25) (layer F.Cu) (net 1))
 (segment (start 105.564988 98.379988) (end 106.963057 98.379989) (width 0.25) (layer F.Cu) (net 1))
 (segment (start 109.299267 100.785001) (end 118.134999 100.785001) (width 0.25) (layer F.Cu) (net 1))
 (via (at 118.85 102.95) (size 0.8) (drill 0.4) (layers F.Cu B.Cu) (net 8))
 (via (at 121.98501 102.95) (size 0.8) (drill 0.4) (layers F.Cu B.Cu) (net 8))
 (segment (start 122.3 104.3) (end 122.3 103.26499) (width 0.25) (layer F.Cu) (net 8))
 (segment (start 118.85 102.95) (end 121.98501 102.95) (width 0.25) (layer B.Cu) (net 8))
 (segment (start 122.3 103.26499) (end 121.98501 102.95) (width 0.25) (layer F.Cu) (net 8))
 (segment (start 108.608001 100.814999) (end 110.743002 102.95) (width 0.25) (layer F.Cu) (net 8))
 (segment (start 110.743002 102.95) (end 118.284315 102.95) (width 0.25) (layer F.Cu) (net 8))
 (segment (start 107.829989 100.288055) (end 108.356933 100.814999) (width 0.25) (layer F.Cu) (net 8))
 (segment (start 101.52 96.875) (end 101.52 98.125) (width 0.25) (layer F.Cu) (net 8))
 (segment (start 108.356933 100.814999) (end 108.608001 100.814999) (width 0.25) (layer F.Cu) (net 8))
 (segment (start 118.284315 102.95) (end 118.85 102.95) (width 0.25) (layer F.Cu) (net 8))
 (segment (start 106.751803 98.889999) (end 107.829988 99.968184) (width 0.25) (layer F.Cu) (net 8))
 (segment (start 107.829988 99.968184) (end 107.829989 100.288055) (width 0.25) (layer F.Cu) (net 8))
 (segment (start 102.284998 98.889998) (end 106.751803 98.889999) (width 0.25) (layer F.Cu) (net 8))
 (segment (start 101.52 98.125) (end 102.284998 98.889998) (width 0.25) (layer F.Cu) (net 8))
 (segment (start 121.2 101.03) (end 122.08 100.15) (width 0.25) (layer F.Cu) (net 3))
 (segment (start 121.2 104.3) (end 121.2 101.03) (width 0.25) (layer F.Cu) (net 3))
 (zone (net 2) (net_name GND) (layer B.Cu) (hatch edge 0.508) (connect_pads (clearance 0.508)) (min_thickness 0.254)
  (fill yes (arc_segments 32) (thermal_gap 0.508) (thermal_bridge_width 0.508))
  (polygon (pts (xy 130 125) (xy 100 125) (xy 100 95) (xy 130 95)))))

